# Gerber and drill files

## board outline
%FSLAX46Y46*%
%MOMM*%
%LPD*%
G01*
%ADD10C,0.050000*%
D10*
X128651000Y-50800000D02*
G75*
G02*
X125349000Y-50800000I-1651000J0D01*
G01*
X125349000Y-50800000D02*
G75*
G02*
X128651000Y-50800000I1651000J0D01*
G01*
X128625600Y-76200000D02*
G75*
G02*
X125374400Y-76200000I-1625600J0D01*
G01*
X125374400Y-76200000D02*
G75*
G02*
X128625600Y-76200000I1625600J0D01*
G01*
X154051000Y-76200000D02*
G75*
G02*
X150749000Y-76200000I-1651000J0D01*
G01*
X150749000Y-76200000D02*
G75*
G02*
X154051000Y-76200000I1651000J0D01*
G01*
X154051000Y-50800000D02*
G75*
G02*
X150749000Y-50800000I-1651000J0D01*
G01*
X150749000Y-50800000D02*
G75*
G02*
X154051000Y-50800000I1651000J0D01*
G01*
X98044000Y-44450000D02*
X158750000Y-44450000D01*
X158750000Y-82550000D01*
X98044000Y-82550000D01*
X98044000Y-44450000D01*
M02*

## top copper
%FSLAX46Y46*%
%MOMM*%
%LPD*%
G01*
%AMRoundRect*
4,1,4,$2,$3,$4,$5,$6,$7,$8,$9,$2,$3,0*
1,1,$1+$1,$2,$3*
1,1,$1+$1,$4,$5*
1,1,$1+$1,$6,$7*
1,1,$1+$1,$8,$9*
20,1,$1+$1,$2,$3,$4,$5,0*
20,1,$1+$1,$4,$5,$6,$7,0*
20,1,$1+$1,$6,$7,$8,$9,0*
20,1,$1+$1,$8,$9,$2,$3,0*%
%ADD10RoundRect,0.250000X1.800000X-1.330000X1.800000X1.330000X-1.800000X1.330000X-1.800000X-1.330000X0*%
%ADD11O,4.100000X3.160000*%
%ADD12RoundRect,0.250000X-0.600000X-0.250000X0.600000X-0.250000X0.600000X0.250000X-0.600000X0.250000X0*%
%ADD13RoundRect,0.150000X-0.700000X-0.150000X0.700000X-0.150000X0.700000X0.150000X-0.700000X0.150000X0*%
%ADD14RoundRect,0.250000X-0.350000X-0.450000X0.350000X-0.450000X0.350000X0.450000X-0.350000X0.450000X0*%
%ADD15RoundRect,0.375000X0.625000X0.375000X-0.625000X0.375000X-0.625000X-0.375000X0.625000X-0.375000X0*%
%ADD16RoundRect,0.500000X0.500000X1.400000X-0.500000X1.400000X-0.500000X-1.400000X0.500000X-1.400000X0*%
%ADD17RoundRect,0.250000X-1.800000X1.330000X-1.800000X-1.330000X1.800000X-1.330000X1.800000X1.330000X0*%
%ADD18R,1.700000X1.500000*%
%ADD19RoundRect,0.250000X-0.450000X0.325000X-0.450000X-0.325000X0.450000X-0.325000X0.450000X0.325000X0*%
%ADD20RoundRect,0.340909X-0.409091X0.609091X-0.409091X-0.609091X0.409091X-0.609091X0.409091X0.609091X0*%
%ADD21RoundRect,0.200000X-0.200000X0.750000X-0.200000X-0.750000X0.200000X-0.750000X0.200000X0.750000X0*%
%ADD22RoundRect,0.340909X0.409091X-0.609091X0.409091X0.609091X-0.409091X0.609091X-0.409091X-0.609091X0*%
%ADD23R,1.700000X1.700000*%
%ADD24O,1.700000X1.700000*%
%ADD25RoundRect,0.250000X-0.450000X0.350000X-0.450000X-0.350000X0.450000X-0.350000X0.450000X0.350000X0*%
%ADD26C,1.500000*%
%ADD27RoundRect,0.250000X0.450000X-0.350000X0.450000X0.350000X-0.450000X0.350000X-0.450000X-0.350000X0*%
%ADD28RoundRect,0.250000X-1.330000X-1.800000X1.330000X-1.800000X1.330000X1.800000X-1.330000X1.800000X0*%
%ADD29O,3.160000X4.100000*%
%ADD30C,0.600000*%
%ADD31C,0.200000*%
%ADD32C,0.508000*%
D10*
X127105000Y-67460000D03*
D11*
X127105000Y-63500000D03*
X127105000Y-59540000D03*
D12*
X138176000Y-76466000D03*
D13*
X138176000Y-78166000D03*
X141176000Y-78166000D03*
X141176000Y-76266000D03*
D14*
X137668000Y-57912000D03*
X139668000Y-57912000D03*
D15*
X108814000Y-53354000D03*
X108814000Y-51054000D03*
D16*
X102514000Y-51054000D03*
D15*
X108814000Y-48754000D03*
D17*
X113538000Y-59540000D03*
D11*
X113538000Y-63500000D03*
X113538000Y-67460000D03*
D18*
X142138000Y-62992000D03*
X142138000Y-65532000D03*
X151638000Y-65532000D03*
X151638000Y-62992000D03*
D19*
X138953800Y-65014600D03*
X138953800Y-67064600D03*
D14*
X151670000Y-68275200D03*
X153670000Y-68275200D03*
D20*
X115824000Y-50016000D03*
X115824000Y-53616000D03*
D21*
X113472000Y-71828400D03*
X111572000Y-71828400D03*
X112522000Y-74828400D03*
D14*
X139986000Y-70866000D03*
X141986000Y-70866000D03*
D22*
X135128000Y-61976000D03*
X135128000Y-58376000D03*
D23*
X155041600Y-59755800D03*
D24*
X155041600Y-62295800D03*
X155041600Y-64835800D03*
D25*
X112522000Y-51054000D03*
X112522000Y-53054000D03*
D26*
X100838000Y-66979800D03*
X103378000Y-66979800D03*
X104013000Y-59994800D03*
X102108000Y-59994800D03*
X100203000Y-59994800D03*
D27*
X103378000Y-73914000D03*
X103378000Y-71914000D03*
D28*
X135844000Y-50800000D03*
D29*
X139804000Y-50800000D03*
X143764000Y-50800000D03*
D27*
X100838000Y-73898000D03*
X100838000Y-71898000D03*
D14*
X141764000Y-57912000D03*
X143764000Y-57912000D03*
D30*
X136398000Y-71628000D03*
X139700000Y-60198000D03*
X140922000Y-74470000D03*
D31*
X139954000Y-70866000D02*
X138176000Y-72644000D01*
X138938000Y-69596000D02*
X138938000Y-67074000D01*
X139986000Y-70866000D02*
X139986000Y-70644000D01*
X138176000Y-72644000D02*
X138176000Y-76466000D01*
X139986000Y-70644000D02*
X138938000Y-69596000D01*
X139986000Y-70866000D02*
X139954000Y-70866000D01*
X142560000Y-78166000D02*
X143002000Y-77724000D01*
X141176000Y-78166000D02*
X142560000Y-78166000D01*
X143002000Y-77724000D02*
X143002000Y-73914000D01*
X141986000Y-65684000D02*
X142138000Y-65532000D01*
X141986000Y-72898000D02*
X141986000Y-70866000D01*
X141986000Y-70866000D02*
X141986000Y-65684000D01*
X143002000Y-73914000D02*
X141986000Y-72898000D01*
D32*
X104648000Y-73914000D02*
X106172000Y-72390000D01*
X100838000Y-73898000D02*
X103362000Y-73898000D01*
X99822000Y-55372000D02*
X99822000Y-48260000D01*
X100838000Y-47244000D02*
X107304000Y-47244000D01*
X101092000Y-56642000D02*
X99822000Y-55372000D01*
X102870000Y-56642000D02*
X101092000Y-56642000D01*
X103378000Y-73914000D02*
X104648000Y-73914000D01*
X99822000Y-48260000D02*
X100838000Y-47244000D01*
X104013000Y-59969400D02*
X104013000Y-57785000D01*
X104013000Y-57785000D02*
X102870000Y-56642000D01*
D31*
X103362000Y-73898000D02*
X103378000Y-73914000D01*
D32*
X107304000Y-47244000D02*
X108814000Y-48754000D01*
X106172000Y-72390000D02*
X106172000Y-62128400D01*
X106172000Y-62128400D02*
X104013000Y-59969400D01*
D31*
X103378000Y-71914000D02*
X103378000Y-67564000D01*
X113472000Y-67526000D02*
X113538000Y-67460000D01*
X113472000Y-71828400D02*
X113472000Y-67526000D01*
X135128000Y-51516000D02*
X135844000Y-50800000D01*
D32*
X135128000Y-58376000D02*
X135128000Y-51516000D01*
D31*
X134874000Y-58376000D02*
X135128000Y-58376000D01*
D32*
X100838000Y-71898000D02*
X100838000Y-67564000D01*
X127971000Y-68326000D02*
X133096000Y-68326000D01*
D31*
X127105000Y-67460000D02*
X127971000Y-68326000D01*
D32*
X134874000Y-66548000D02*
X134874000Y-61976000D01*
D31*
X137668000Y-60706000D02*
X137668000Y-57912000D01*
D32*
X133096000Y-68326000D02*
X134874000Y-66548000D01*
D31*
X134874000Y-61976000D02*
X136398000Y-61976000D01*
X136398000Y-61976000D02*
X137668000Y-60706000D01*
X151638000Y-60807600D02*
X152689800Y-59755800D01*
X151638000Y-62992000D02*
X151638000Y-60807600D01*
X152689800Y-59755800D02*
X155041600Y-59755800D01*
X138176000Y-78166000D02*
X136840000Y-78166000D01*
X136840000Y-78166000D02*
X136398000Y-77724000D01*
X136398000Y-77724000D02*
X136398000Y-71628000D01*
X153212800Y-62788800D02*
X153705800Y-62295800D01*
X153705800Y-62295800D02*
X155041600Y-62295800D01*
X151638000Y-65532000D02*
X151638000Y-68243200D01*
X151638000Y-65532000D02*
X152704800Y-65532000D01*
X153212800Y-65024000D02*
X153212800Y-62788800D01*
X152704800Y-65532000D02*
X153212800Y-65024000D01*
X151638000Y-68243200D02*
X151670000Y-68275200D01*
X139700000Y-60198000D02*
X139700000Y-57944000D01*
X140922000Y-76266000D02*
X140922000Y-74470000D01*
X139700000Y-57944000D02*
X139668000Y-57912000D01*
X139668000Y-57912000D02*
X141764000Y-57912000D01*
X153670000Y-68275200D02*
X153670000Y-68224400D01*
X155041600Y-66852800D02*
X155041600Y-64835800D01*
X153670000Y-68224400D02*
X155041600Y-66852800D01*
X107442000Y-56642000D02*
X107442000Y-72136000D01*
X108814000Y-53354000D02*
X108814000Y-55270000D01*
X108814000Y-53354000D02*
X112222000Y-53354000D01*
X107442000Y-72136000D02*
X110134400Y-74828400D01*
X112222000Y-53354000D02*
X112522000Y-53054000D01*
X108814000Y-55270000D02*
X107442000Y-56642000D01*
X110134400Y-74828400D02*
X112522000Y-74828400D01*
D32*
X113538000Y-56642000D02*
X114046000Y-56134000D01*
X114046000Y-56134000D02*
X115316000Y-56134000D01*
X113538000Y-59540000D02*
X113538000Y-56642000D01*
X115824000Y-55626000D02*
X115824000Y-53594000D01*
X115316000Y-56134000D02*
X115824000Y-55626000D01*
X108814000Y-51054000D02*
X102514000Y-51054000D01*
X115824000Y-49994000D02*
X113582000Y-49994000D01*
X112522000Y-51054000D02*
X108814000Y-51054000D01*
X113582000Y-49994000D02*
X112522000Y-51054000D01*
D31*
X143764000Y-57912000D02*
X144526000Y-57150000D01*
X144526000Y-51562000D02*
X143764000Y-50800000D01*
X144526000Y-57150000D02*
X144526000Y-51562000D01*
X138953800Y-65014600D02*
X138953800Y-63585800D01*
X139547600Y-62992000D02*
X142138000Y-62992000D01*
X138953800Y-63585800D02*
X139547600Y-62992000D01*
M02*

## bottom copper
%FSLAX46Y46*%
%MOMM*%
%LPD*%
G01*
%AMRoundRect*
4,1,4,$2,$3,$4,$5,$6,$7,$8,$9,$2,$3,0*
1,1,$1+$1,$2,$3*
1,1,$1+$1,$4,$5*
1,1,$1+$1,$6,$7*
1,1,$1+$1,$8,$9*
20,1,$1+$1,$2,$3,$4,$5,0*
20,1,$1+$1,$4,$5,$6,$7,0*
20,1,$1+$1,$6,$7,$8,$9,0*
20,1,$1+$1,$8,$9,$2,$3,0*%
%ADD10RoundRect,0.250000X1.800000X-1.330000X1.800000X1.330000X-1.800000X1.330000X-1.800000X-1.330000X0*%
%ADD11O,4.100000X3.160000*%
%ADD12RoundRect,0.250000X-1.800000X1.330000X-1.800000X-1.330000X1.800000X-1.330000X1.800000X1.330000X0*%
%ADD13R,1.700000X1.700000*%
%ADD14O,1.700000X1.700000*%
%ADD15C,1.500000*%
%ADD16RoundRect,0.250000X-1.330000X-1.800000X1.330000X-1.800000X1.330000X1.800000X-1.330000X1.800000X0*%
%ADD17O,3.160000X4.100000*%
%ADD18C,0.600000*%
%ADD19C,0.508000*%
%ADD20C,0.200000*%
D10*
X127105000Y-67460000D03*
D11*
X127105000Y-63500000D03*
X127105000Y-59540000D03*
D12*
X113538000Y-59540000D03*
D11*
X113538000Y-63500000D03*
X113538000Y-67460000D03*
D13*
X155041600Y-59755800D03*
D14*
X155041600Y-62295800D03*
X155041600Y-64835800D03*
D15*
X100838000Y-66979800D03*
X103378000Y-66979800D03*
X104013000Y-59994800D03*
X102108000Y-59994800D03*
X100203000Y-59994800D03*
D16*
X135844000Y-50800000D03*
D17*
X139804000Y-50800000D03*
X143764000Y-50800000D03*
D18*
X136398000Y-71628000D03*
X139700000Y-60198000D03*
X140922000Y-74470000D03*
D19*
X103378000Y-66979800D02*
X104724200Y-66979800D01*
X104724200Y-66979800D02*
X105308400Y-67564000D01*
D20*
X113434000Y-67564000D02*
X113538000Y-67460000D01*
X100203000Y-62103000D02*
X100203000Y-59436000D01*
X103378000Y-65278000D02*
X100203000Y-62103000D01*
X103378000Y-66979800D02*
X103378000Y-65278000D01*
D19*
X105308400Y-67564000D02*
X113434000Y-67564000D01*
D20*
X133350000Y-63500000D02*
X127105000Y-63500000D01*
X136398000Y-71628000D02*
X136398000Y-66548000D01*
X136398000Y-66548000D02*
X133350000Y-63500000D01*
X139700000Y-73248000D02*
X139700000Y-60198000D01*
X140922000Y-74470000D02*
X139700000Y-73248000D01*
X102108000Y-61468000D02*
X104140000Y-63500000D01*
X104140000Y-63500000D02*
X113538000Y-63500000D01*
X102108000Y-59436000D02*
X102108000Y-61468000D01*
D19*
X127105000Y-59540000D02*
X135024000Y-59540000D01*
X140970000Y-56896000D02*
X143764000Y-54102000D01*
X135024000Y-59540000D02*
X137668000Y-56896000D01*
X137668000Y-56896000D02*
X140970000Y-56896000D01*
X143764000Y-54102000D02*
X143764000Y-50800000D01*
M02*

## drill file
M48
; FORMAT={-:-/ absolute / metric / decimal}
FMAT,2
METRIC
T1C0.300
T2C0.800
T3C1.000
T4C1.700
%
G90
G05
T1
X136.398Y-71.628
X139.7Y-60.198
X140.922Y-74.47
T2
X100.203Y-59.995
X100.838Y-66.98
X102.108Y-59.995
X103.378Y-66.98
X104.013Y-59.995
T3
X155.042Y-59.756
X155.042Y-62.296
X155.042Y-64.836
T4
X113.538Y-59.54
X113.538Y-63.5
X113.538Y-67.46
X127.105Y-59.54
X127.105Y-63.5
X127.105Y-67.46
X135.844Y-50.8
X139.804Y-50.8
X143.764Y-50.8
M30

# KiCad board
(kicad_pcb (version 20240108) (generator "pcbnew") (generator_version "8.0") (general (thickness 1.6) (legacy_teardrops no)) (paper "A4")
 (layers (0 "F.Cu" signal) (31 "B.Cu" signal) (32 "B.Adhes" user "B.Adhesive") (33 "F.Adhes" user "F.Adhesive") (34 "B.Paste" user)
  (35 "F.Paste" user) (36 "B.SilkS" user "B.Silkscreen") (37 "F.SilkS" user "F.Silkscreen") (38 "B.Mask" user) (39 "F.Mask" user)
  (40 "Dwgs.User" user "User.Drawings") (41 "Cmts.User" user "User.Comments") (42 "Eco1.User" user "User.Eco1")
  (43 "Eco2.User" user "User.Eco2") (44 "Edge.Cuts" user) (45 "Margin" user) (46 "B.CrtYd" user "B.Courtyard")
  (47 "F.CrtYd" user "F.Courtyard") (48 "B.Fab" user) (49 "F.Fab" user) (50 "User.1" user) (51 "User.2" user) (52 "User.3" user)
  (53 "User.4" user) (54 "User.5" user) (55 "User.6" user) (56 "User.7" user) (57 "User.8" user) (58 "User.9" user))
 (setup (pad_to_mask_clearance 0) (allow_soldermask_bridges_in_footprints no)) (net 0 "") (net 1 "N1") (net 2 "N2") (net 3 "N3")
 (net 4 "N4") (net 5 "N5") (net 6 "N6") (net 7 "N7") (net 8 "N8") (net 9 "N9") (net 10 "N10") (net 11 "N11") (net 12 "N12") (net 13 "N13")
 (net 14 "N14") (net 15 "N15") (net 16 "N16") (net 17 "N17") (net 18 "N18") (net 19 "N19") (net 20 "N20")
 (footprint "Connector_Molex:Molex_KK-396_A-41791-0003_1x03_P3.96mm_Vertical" (layer "F.Cu") (at 127.105 67.46 90)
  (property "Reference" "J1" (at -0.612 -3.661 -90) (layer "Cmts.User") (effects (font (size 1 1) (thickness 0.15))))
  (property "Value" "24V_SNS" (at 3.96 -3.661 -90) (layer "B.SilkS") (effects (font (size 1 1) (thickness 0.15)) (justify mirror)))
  (pad "1" thru_hole roundrect (at 0 0 90) (size 3.16 4.1) (drill 1.7) (layers "*.Cu" "*.Mask") (remove_unused_layers no)
   (roundrect_rratio 0.079114) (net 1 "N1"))
  (pad "2" thru_hole oval (at 3.96 0 90) (size 3.16 4.1) (drill 1.7) (layers "*.Cu" "*.Mask") (remove_unused_layers no) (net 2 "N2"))
  (pad "3" thru_hole oval (at 7.92 0 90) (size 3.16 4.1) (drill 1.7) (layers "*.Cu" "*.Mask") (remove_unused_layers no) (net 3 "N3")))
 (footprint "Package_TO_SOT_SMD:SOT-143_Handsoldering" (layer "F.Cu") (at 139.676 77.216)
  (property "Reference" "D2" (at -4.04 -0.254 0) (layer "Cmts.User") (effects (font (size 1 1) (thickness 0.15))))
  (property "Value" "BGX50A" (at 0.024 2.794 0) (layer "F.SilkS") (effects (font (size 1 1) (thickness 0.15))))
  (pad "1" smd roundrect (at -1.5 -0.75) (size 1.7 1) (layers "F.Cu" "F.Paste" "F.Mask") (roundrect_rratio 0.25) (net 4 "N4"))
  (pad "2" smd roundrect (at -1.5 0.95) (size 1.7 0.6) (layers "F.Cu" "F.Paste" "F.Mask") (roundrect_rratio 0.25) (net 2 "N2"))
  (pad "3" smd roundrect (at 1.5 0.95) (size 1.7 0.6) (layers "F.Cu" "F.Paste" "F.Mask") (roundrect_rratio 0.25) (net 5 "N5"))
  (pad "4" smd roundrect (at 1.5 -0.95) (size 1.7 0.6) (layers "F.Cu" "F.Paste" "F.Mask") (roundrect_rratio 0.25) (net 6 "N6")))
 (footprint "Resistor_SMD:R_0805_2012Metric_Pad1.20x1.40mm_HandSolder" (layer "F.Cu") (at 138.668 57.912)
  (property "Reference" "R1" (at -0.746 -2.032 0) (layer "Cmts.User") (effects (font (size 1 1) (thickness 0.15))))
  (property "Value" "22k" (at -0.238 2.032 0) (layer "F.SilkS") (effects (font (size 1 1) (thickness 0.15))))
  (pad "1" smd roundrect (at -1 0) (size 1.2 1.4) (layers "F.Cu" "F.Paste" "F.Mask") (roundrect_rratio 0.208333) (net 1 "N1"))
  (pad "2" smd roundrect (at 1 0) (size 1.2 1.4) (layers "F.Cu" "F.Paste" "F.Mask") (roundrect_rratio 0.208333) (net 6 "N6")))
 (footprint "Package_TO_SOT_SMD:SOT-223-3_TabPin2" (layer "F.Cu") (at 105.664 51.054 180)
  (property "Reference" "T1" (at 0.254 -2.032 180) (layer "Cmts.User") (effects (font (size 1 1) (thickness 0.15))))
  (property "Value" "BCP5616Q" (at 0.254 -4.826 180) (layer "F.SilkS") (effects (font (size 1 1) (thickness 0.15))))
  (pad "1" smd roundrect (at -3.15 -2.3 180) (size 2 1.5) (layers "F.Cu" "F.Paste" "F.Mask") (roundrect_rratio 0.25) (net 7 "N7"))
  (pad "2" smd roundrect (at -3.15 0 180) (size 2 1.5) (layers "F.Cu" "F.Paste" "F.Mask") (roundrect_rratio 0.25) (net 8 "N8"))
  (pad "2" smd roundrect (at 3.15 0 180) (size 2 3.8) (layers "F.Cu" "F.Paste" "F.Mask") (roundrect_rratio 0.25) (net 8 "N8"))
  (pad "3" smd roundrect (at -3.15 2.3 180) (size 2 1.5) (layers "F.Cu" "F.Paste" "F.Mask") (roundrect_rratio 0.25) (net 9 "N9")))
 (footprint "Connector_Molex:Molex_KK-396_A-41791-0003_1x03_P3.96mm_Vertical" (layer "F.Cu") (at 113.538 59.54 -90)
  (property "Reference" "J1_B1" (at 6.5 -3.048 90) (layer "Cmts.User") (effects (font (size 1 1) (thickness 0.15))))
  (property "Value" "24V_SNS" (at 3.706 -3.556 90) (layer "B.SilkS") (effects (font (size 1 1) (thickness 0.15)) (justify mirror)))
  (pad "1" thru_hole roundrect (at 0 0 270) (size 3.16 4.1) (drill 1.7) (layers "*.Cu" "*.Mask") (remove_unused_layers no)
   (roundrect_rratio 0.079114) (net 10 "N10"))
  (pad "2" thru_hole oval (at 3.96 0 270) (size 3.16 4.1) (drill 1.7) (layers "*.Cu" "*.Mask") (remove_unused_layers no) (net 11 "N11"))
  (pad "3" thru_hole oval (at 7.92 0 270) (size 3.16 4.1) (drill 1.7) (layers "*.Cu" "*.Mask") (remove_unused_layers no) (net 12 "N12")))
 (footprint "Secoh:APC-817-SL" (layer "F.Cu") (at 146.888 64.262 -90)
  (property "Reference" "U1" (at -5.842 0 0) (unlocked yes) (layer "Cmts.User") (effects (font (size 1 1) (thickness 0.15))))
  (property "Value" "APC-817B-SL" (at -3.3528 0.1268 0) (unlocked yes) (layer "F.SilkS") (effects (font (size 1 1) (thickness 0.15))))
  (pad "1" smd rect (at -1.27 4.75 270) (size 1.5 1.7) (layers "F.Cu" "F.Paste" "F.Mask") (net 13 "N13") (thermal_bridge_angle 45))
  (pad "2" smd rect (at 1.27 4.75 270) (size 1.5 1.7) (layers "F.Cu" "F.Paste" "F.Mask") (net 5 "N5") (thermal_bridge_angle 45))
  (pad "3" smd rect (at 1.27 -4.75 270) (size 1.5 1.7) (layers "F.Cu" "F.Paste" "F.Mask") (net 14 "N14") (thermal_bridge_angle 45))
  (pad "4" smd rect (at -1.27 -4.75 270) (size 1.5 1.7) (layers "F.Cu" "F.Paste" "F.Mask") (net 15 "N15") (thermal_bridge_angle 45)))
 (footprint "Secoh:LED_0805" (layer "F.Cu") (at 138.938 66.049 -90)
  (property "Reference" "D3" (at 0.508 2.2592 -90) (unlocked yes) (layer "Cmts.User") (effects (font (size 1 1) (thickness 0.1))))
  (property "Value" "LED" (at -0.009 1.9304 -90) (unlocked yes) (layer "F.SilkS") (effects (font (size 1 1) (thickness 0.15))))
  (pad "1" smd roundrect (at -1.0344 -0.0158 270) (size 1.15 1.4) (layers "F.Cu" "F.Paste" "F.Mask") (roundrect_rratio 0.217391)
   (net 13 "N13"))
  (pad "2" smd roundrect (at 1.0156 -0.0158 270) (size 1.15 1.4) (layers "F.Cu" "F.Paste" "F.Mask") (roundrect_rratio 0.217391) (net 4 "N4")))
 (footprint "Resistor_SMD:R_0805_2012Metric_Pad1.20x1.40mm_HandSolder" (layer "F.Cu") (at 152.67 68.2752)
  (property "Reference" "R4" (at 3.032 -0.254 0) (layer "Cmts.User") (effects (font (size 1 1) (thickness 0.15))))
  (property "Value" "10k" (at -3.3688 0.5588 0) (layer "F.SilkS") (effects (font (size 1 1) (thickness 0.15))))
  (pad "1" smd roundrect (at -1 0) (size 1.2 1.4) (layers "F.Cu" "F.Paste" "F.Mask") (roundrect_rratio 0.208333) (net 14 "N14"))
  (pad "2" smd roundrect (at 1 0) (size 1.2 1.4) (layers "F.Cu" "F.Paste" "F.Mask") (roundrect_rratio 0.208333) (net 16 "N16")))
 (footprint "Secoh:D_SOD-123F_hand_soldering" (layer "F.Cu") (at 115.824 51.816 -90)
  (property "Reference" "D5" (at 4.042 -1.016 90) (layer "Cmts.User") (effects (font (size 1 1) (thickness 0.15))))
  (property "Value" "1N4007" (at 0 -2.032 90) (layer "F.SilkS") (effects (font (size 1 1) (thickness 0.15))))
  (pad "1" smd roundrect (at -1.8 0 270) (size 1.9 1.5) (layers "F.Cu" "F.Paste" "F.Mask") (roundrect_rratio 0.2272727273) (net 8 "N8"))
  (pad "2" smd roundrect (at 1.8 0 270) (size 1.9 1.5) (layers "F.Cu" "F.Paste" "F.Mask") (roundrect_rratio 0.2272727273) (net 10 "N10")))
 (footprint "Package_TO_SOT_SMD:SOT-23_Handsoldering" (layer "F.Cu") (at 112.522 73.3284 -90)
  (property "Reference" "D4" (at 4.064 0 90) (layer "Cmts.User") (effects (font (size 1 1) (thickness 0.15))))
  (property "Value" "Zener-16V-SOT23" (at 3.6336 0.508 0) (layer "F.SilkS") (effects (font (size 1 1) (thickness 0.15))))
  (pad "1" smd roundrect (at -1.5 -0.95 270) (size 1.9 0.8) (layers "F.Cu" "F.Paste" "F.Mask") (roundrect_rratio 0.25) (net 12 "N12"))
  (pad "2" smd roundrect (at -1.5 0.95 270) (size 1.9 0.8) (layers "F.Cu" "F.Paste" "F.Mask") (roundrect_rratio 0.25) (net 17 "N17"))
  (pad "3" smd roundrect (at 1.5 0 270) (size 1.9 0.8) (layers "F.Cu" "F.Paste" "F.Mask") (roundrect_rratio 0.25) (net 7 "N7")))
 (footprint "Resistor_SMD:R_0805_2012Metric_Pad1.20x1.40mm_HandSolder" (layer "F.Cu") (at 140.986 70.866)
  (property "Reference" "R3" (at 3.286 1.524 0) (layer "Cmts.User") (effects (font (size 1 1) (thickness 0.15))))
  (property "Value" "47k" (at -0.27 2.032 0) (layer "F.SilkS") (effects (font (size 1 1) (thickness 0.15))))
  (pad "1" smd roundrect (at -1 0) (size 1.2 1.4) (layers "F.Cu" "F.Paste" "F.Mask") (roundrect_rratio 0.208333) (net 4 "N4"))
  (pad "2" smd roundrect (at 1 0) (size 1.2 1.4) (layers "F.Cu" "F.Paste" "F.Mask") (roundrect_rratio 0.208333) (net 5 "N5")))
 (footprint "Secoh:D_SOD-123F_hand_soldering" (layer "F.Cu") (at 135.128 60.176 90)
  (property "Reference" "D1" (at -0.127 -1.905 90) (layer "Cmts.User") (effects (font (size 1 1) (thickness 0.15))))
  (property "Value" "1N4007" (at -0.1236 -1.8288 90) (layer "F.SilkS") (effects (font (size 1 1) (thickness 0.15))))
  (pad "1" smd roundrect (at -1.8 0 90) (size 1.9 1.5) (layers "F.Cu" "F.Paste" "F.Mask") (roundrect_rratio 0.2272727273) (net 1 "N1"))
  (pad "2" smd roundrect (at 1.8 0 90) (size 1.9 1.5) (layers "F.Cu" "F.Paste" "F.Mask") (roundrect_rratio 0.2272727273) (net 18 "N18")))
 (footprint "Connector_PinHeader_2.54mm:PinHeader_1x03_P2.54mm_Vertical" (layer "F.Cu") (at 155.0416 59.7558)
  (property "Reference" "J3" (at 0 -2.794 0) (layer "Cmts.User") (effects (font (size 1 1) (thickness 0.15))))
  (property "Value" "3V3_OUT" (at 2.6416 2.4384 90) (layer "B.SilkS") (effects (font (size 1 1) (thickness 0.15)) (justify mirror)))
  (pad "1" thru_hole rect (at 0 0) (size 1.7 1.7) (drill 1) (layers "*.Cu" "*.Mask") (remove_unused_layers no) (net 15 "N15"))
  (pad "2" thru_hole oval (at 0 2.54) (size 1.7 1.7) (drill 1) (layers "*.Cu" "*.Mask") (remove_unused_layers no) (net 14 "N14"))
  (pad "3" thru_hole oval (at 0 5.08) (size 1.7 1.7) (drill 1) (layers "*.Cu" "*.Mask") (remove_unused_layers no) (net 16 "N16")))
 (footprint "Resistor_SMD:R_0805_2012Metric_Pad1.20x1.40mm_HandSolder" (layer "F.Cu") (at 112.522 52.054 -90)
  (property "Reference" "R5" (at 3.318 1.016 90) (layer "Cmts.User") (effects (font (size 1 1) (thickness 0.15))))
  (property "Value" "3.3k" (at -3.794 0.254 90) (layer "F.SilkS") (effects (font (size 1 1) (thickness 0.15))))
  (pad "1" smd roundrect (at -1 0 270) (size 1.2 1.4) (layers "F.Cu" "F.Paste" "F.Mask") (roundrect_rratio 0.208333) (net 8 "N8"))
  (pad "2" smd roundrect (at 1 0 270) (size 1.2 1.4) (layers "F.Cu" "F.Paste" "F.Mask") (roundrect_rratio 0.208333) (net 7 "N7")))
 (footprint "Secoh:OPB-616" (layer "F.Cu") (at 102.108 63.5)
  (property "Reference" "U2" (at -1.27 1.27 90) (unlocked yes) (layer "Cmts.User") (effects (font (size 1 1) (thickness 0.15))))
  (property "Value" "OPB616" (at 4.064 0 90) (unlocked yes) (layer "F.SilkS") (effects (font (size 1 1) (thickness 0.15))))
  (pad "1" thru_hole circle (at -1.27 3.4798) (size 1.5 1.5) (drill 0.8) (layers "*.Cu" "*.Mask") (remove_unused_layers no) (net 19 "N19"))
  (pad "2" thru_hole circle (at 1.27 3.4798) (size 1.5 1.5) (drill 0.8) (layers "*.Cu" "*.Mask") (remove_unused_layers no) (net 12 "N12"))
  (pad "3" thru_hole circle (at 1.905 -3.5052) (size 1.5 1.5) (drill 0.8) (layers "*.Cu" "*.Mask") (remove_unused_layers no) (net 9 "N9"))
  (pad "4" thru_hole circle (at 0 -3.5052) (size 1.5 1.5) (drill 0.8) (layers "*.Cu" "*.Mask") (remove_unused_layers no) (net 11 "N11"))
  (pad "5" thru_hole circle (at -1.905 -3.5052) (size 1.5 1.5) (drill 0.8) (layers "*.Cu" "*.Mask") (remove_unused_layers no) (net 12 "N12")))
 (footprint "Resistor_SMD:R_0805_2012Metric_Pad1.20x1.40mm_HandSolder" (layer "F.Cu") (at 103.378 72.914 90)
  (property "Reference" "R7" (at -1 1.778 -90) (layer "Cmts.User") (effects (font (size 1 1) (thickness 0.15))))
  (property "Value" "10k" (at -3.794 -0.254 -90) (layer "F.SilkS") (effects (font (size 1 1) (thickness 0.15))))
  (pad "1" smd roundrect (at -1 0 90) (size 1.2 1.4) (layers "F.Cu" "F.Paste" "F.Mask") (roundrect_rratio 0.208333) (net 9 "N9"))
  (pad "2" smd roundrect (at 1 0 90) (size 1.2 1.4) (layers "F.Cu" "F.Paste" "F.Mask") (roundrect_rratio 0.208333) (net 12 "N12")))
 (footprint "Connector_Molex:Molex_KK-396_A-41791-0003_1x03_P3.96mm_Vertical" (layer "F.Cu") (at 135.844 50.8)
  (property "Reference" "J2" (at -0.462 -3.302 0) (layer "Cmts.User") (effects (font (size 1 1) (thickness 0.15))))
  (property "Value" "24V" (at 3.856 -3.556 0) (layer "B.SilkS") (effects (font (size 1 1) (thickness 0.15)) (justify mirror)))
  (pad "1" thru_hole roundrect (at 0 0) (size 3.16 4.1) (drill 1.7) (layers "*.Cu" "*.Mask") (remove_unused_layers no)
   (roundrect_rratio 0.079114) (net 18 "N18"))
  (pad "2" thru_hole oval (at 3.96 0) (size 3.16 4.1) (drill 1.7) (layers "*.Cu" "*.Mask") (remove_unused_layers no) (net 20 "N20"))
  (pad "3" thru_hole oval (at 7.92 0) (size 3.16 4.1) (drill 1.7) (layers "*.Cu" "*.Mask") (remove_unused_layers no) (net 3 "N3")))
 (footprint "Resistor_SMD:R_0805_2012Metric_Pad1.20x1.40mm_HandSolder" (layer "F.Cu") (at 100.838 72.898 90)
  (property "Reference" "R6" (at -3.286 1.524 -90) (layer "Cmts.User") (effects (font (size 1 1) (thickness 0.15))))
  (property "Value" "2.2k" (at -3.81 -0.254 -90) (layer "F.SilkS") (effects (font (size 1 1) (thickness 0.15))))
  (pad "1" smd roundrect (at -1 0 90) (size 1.2 1.4) (layers "F.Cu" "F.Paste" "F.Mask") (roundrect_rratio 0.208333) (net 9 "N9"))
  (pad "2" smd roundrect (at 1 0 90) (size 1.2 1.4) (layers "F.Cu" "F.Paste" "F.Mask") (roundrect_rratio 0.208333) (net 19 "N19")))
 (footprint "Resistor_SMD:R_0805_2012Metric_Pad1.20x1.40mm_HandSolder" (layer "F.Cu") (at 142.764 57.912)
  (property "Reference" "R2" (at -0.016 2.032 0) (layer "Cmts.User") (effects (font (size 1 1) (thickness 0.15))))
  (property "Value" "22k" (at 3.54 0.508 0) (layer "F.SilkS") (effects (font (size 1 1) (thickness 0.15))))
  (pad "1" smd roundrect (at -1 0) (size 1.2 1.4) (layers "F.Cu" "F.Paste" "F.Mask") (roundrect_rratio 0.208333) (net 6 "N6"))
  (pad "2" smd roundrect (at 1 0) (size 1.2 1.4) (layers "F.Cu" "F.Paste" "F.Mask") (roundrect_rratio 0.208333) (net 3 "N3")))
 (gr_circle (center 127 50.8) (end 128.651 50.8) (stroke (width 0.05) (type default)) (fill none) (layer "Edge.Cuts"))
 (gr_circle (center 127 76.2) (end 128.6256 76.2) (stroke (width 0.05) (type default)) (fill none) (layer "Edge.Cuts"))
 (gr_circle (center 152.4 76.2) (end 154.051 76.2) (stroke (width 0.05) (type default)) (fill none) (layer "Edge.Cuts"))
 (gr_circle (center 152.4 50.8) (end 154.051 50.8) (stroke (width 0.05) (type default)) (fill none) (layer "Edge.Cuts"))
 (gr_rect (start 98.044 44.45) (end 158.75 82.55) (stroke (width 0.05) (type default)) (fill none) (layer "Edge.Cuts"))
 (segment (start 139.954 70.866) (end 138.176 72.644) (width 0.2) (layer "F.Cu") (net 4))
 (segment (start 138.938 69.596) (end 138.938 67.074) (width 0.2) (layer "F.Cu") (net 4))
 (segment (start 139.986 70.866) (end 139.986 70.644) (width 0.2) (layer "F.Cu") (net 4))
 (segment (start 138.176 72.644) (end 138.176 76.466) (width 0.2) (layer "F.Cu") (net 4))
 (segment (start 139.986 70.644) (end 138.938 69.596) (width 0.2) (layer "F.Cu") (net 4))
 (segment (start 139.986 70.866) (end 139.954 70.866) (width 0.2) (layer "F.Cu") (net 4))
 (segment (start 142.56 78.166) (end 143.002 77.724) (width 0.2) (layer "F.Cu") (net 5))
 (segment (start 141.176 78.166) (end 142.56 78.166) (width 0.2) (layer "F.Cu") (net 5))
 (segment (start 143.002 77.724) (end 143.002 73.914) (width 0.2) (layer "F.Cu") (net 5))
 (segment (start 141.986 65.684) (end 142.138 65.532) (width 0.2) (layer "F.Cu") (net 5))
 (segment (start 141.986 72.898) (end 141.986 70.866) (width 0.2) (layer "F.Cu") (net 5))
 (segment (start 141.986 70.866) (end 141.986 65.684) (width 0.2) (layer "F.Cu") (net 5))
 (segment (start 143.002 73.914) (end 141.986 72.898) (width 0.2) (layer "F.Cu") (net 5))
 (segment (start 104.648 73.914) (end 106.172 72.39) (width 0.508) (layer "F.Cu") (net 9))
 (segment (start 100.838 73.898) (end 103.362 73.898) (width 0.508) (layer "F.Cu") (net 9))
 (segment (start 99.822 55.372) (end 99.822 48.26) (width 0.508) (layer "F.Cu") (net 9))
 (segment (start 100.838 47.244) (end 107.304 47.244) (width 0.508) (layer "F.Cu") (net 9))
 (segment (start 101.092 56.642) (end 99.822 55.372) (width 0.508) (layer "F.Cu") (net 9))
 (segment (start 102.87 56.642) (end 101.092 56.642) (width 0.508) (layer "F.Cu") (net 9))
 (segment (start 103.378 73.914) (end 104.648 73.914) (width 0.508) (layer "F.Cu") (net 9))
 (segment (start 99.822 48.26) (end 100.838 47.244) (width 0.508) (layer "F.Cu") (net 9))
 (segment (start 104.013 59.9694) (end 104.013 57.785) (width 0.508) (layer "F.Cu") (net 9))
 (segment (start 104.013 57.785) (end 102.87 56.642) (width 0.508) (layer "F.Cu") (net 9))
 (segment (start 103.362 73.898) (end 103.378 73.914) (width 0.2) (layer "F.Cu") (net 9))
 (segment (start 107.304 47.244) (end 108.814 48.754) (width 0.508) (layer "F.Cu") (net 9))
 (segment (start 106.172 72.39) (end 106.172 62.1284) (width 0.508) (layer "F.Cu") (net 9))
 (segment (start 106.172 62.1284) (end 104.013 59.9694) (width 0.508) (layer "F.Cu") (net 9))
 (segment (start 103.378 71.914) (end 103.378 67.564) (width 0.2) (layer "F.Cu") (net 12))
 (segment (start 113.472 67.526) (end 113.538 67.46) (width 0.2) (layer "F.Cu") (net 12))
 (segment (start 113.472 71.8284) (end 113.472 67.526) (width 0.2) (layer "F.Cu") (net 12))
 (segment (start 103.378 66.9798) (end 104.7242 66.9798) (width 0.508) (layer "B.Cu") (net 12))
 (segment (start 104.7242 66.9798) (end 105.3084 67.564) (width 0.508) (layer "B.Cu") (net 12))
 (segment (start 113.434 67.564) (end 113.538 67.46) (width 0.2) (layer "B.Cu") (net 12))
 (segment (start 100.203 62.103) (end 100.203 59.436) (width 0.2) (layer "B.Cu") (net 12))
 (segment (start 103.378 65.278) (end 100.203 62.103) (width 0.2) (layer "B.Cu") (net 12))
 (segment (start 103.378 66.9798) (end 103.378 65.278) (width 0.2) (layer "B.Cu") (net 12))
 (segment (start 105.3084 67.564) (end 113.434 67.564) (width 0.508) (layer "B.Cu") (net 12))
 (segment (start 135.128 51.516) (end 135.844 50.8) (width 0.2) (layer "F.Cu") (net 18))
 (segment (start 135.128 58.376) (end 135.128 51.516) (width 0.508) (layer "F.Cu") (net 18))
 (segment (start 134.874 58.376) (end 135.128 58.376) (width 0.2) (layer "F.Cu") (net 18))
 (segment (start 100.838 71.898) (end 100.838 67.564) (width 0.508) (layer "F.Cu") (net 19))
 (segment (start 127.971 68.326) (end 133.096 68.326) (width 0.508) (layer "F.Cu") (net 1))
 (segment (start 127.105 67.46) (end 127.971 68.326) (width 0.2) (layer "F.Cu") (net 1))
 (segment (start 134.874 66.548) (end 134.874 61.976) (width 0.508) (layer "F.Cu") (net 1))
 (segment (start 137.668 60.706) (end 137.668 57.912) (width 0.2) (layer "F.Cu") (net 1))
 (segment (start 133.096 68.326) (end 134.874 66.548) (width 0.508) (layer "F.Cu") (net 1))
 (segment (start 134.874 61.976) (end 136.398 61.976) (width 0.2) (layer "F.Cu") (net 1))
 (segment (start 136.398 61.976) (end 137.668 60.706) (width 0.2) (layer "F.Cu") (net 1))
 (segment (start 151.638 60.8076) (end 152.6898 59.7558) (width 0.2) (layer "F.Cu") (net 15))
 (segment (start 151.638 62.992) (end 151.638 60.8076) (width 0.2) (layer "F.Cu") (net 15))
 (segment (start 152.6898 59.7558) (end 155.0416 59.7558) (width 0.2) (layer "F.Cu") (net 15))
 (segment (start 138.176 78.166) (end 136.84 78.166) (width 0.2) (layer "F.Cu") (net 2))
 (segment (start 136.84 78.166) (end 136.398 77.724) (width 0.2) (layer "F.Cu") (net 2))
 (segment (start 136.398 77.724) (end 136.398 71.628) (width 0.2) (layer "F.Cu") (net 2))
 (via (at 136.398 71.628) (size 0.6) (drill 0.3) (layers "F.Cu" "B.Cu") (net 2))
 (segment (start 133.35 63.5) (end 127.105 63.5) (width 0.2) (layer "B.Cu") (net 2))
 (segment (start 136.398 71.628) (end 136.398 66.548) (width 0.2) (layer "B.Cu") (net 2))
 (segment (start 136.398 66.548) (end 133.35 63.5) (width 0.2) (layer "B.Cu") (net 2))
 (segment (start 153.2128 62.7888) (end 153.7058 62.2958) (width 0.2) (layer "F.Cu") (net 14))
 (segment (start 153.7058 62.2958) (end 155.0416 62.2958) (width 0.2) (layer "F.Cu") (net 14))
 (segment (start 151.638 65.532) (end 151.638 68.2432) (width 0.2) (layer "F.Cu") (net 14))
 (segment (start 151.638 65.532) (end 152.7048 65.532) (width 0.2) (layer "F.Cu") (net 14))
 (segment (start 153.2128 65.024) (end 153.2128 62.7888) (width 0.2) (layer "F.Cu") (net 14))
 (segment (start 152.7048 65.532) (end 153.2128 65.024) (width 0.2) (layer "F.Cu") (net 14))
 (segment (start 151.638 68.2432) (end 151.67 68.2752) (width 0.2) (layer "F.Cu") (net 14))
 (segment (start 139.7 60.198) (end 139.7 57.944) (width 0.2) (layer "F.Cu") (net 6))
 (segment (start 140.922 76.266) (end 140.922 74.47) (width 0.2) (layer "F.Cu") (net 6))
 (segment (start 139.7 57.944) (end 139.668 57.912) (width 0.2) (layer "F.Cu") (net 6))
 (segment (start 139.668 57.912) (end 141.764 57.912) (width 0.2) (layer "F.Cu") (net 6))
 (via (at 139.7 60.198) (size 0.6) (drill 0.3) (layers "F.Cu" "B.Cu") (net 6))
 (via (at 140.922 74.47) (size 0.6) (drill 0.3) (layers "F.Cu" "B.Cu") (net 6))
 (segment (start 139.7 73.248) (end 139.7 60.198) (width 0.2) (layer "B.Cu") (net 6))
 (segment (start 140.922 74.47) (end 139.7 73.248) (width 0.2) (layer "B.Cu") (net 6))
 (segment (start 153.67 68.2752) (end 153.67 68.2244) (width 0.2) (layer "F.Cu") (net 16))
 (segment (start 155.0416 66.8528) (end 155.0416 64.8358) (width 0.2) (layer "F.Cu") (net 16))
 (segment (start 153.67 68.2244) (end 155.0416 66.8528) (width 0.2) (layer "F.Cu") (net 16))
 (segment (start 107.442 56.642) (end 107.442 72.136) (width 0.2) (layer "F.Cu") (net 7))
 (segment (start 108.814 53.354) (end 108.814 55.27) (width 0.2) (layer "F.Cu") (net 7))
 (segment (start 108.814 53.354) (end 112.222 53.354) (width 0.2) (layer "F.Cu") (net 7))
 (segment (start 107.442 72.136) (end 110.1344 74.8284) (width 0.2) (layer "F.Cu") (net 7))
 (segment (start 112.222 53.354) (end 112.522 53.054) (width 0.2) (layer "F.Cu") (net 7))
 (segment (start 108.814 55.27) (end 107.442 56.642) (width 0.2) (layer "F.Cu") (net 7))
 (segment (start 110.1344 74.8284) (end 112.522 74.8284) (width 0.2) (layer "F.Cu") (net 7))
 (segment (start 102.108 61.468) (end 104.14 63.5) (width 0.2) (layer "B.Cu") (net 11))
 (segment (start 104.14 63.5) (end 113.538 63.5) (width 0.2) (layer "B.Cu") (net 11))
 (segment (start 102.108 59.436) (end 102.108 61.468) (width 0.2) (layer "B.Cu") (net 11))
 (segment (start 113.538 56.642) (end 114.046 56.134) (width 0.508) (layer "F.Cu") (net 10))
 (segment (start 114.046 56.134) (end 115.316 56.134) (width 0.508) (layer "F.Cu") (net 10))
 (segment (start 113.538 59.54) (end 113.538 56.642) (width 0.508) (layer "F.Cu") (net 10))
 (segment (start 115.824 55.626) (end 115.824 53.594) (width 0.508) (layer "F.Cu") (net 10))
 (segment (start 115.316 56.134) (end 115.824 55.626) (width 0.508) (layer "F.Cu") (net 10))
 (segment (start 108.814 51.054) (end 102.514 51.054) (width 0.508) (layer "F.Cu") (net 8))
 (segment (start 115.824 49.994) (end 113.582 49.994) (width 0.508) (layer "F.Cu") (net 8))
 (segment (start 112.522 51.054) (end 108.814 51.054) (width 0.508) (layer "F.Cu") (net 8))
 (segment (start 113.582 49.994) (end 112.522 51.054) (width 0.508) (layer "F.Cu") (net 8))
 (segment (start 143.764 57.912) (end 144.526 57.15) (width 0.2) (layer "F.Cu") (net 3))
 (segment (start 144.526 51.562) (end 143.764 50.8) (width 0.2) (layer "F.Cu") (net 3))
 (segment (start 144.526 57.15) (end 144.526 51.562) (width 0.2) (layer "F.Cu") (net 3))
 (segment (start 127.105 59.54) (end 135.024 59.54) (width 0.508) (layer "B.Cu") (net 3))
 (segment (start 140.97 56.896) (end 143.764 54.102) (width 0.508) (layer "B.Cu") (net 3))
 (segment (start 135.024 59.54) (end 137.668 56.896) (width 0.508) (layer "B.Cu") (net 3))
 (segment (start 137.668 56.896) (end 140.97 56.896) (width 0.508) (layer "B.Cu") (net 3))
 (segment (start 143.764 54.102) (end 143.764 50.8) (width 0.508) (layer "B.Cu") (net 3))
 (segment (start 138.9538 65.0146) (end 138.9538 63.5858) (width 0.2) (layer "F.Cu") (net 13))
 (segment (start 139.5476 62.992) (end 142.138 62.992) (width 0.2) (layer "F.Cu") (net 13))
 (segment (start 138.9538 63.5858) (end 139.5476 62.992) (width 0.2) (layer "F.Cu") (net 13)))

